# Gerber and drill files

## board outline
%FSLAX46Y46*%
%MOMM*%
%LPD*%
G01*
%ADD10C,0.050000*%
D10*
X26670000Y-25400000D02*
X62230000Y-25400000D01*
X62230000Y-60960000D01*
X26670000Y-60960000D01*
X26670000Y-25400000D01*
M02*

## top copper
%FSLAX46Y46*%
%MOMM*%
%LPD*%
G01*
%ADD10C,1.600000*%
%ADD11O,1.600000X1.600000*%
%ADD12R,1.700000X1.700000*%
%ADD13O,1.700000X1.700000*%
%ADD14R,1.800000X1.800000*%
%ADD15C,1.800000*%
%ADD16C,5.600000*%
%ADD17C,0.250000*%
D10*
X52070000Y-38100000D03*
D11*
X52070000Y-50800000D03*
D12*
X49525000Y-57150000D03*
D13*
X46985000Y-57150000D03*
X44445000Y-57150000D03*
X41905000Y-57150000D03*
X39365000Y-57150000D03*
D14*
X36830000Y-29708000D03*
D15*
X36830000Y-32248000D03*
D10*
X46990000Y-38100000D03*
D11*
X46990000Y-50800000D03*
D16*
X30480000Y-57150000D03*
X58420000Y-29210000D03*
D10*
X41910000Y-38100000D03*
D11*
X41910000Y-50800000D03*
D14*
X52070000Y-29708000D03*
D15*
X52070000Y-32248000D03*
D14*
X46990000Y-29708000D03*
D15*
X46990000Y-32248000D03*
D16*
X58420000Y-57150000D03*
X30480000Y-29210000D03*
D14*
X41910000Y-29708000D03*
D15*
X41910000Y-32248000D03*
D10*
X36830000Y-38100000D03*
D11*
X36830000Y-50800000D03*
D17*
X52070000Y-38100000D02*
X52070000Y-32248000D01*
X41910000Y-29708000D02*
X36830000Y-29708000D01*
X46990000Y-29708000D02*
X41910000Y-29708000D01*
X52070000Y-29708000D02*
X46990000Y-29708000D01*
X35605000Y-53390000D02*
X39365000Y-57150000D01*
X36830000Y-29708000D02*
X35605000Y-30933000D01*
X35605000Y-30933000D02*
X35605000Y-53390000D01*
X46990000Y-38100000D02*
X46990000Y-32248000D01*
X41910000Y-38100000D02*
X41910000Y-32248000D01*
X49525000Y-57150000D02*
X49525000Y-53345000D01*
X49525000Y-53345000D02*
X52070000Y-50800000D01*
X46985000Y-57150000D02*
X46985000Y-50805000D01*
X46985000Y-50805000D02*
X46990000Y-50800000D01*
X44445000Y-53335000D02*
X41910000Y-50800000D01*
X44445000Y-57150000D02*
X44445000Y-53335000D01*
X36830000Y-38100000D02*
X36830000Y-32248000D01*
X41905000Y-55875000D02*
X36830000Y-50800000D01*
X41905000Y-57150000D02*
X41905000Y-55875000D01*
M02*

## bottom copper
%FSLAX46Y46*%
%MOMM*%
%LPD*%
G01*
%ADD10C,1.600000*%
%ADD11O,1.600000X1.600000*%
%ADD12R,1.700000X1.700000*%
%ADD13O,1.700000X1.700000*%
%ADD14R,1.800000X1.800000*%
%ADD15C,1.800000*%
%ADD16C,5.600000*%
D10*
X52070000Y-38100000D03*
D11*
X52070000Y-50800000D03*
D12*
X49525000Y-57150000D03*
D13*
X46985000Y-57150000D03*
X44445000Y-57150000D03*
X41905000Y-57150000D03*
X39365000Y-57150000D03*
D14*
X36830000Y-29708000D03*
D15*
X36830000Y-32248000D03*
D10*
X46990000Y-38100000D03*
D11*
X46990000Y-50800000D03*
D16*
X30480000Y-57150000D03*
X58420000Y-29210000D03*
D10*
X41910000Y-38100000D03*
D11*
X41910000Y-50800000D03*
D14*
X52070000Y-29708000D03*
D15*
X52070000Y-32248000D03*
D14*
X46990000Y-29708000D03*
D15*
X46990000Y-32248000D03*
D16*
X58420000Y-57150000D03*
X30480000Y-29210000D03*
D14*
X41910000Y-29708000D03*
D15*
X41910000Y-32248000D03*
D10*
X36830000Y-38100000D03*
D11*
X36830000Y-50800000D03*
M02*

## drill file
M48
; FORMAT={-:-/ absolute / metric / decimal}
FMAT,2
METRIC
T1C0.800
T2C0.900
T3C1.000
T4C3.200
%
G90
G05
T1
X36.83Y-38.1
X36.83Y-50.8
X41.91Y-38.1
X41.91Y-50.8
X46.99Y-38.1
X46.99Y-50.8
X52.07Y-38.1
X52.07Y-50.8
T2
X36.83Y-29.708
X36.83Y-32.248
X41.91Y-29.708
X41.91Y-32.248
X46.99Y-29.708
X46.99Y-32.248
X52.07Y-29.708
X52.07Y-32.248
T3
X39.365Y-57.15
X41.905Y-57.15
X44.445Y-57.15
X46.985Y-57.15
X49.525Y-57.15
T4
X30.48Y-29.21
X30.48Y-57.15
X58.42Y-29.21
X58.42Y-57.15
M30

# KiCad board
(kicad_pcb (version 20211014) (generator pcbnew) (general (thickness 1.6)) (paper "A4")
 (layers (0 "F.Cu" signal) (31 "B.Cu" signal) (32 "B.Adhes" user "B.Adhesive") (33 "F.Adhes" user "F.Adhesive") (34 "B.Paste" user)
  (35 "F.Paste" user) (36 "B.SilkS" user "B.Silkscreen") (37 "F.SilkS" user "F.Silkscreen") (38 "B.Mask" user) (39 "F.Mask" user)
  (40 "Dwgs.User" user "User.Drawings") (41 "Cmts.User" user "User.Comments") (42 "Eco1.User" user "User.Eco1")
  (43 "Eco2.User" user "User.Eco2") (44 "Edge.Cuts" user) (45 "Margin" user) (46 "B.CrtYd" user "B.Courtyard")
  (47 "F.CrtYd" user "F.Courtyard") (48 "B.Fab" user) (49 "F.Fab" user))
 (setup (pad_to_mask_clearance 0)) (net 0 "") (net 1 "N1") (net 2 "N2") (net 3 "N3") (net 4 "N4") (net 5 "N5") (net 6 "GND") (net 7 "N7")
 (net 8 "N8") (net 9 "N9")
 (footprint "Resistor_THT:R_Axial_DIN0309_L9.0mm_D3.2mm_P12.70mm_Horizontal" (layer "F.Cu") (at 52.07 38.1 -90)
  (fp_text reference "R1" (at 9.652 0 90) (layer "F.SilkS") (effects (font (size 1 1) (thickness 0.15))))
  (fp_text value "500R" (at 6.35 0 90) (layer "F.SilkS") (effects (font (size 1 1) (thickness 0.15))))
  (pad "1" thru_hole circle (at 0 0 270) (size 1.6 1.6) (drill 0.8) (layers *.Cu *.Mask) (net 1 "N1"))
  (pad "2" thru_hole oval (at 12.7 0 270) (size 1.6 1.6) (drill 0.8) (layers *.Cu *.Mask) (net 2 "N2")))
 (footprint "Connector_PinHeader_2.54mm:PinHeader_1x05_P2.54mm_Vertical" (layer "F.Cu") (at 49.525 57.15 -90)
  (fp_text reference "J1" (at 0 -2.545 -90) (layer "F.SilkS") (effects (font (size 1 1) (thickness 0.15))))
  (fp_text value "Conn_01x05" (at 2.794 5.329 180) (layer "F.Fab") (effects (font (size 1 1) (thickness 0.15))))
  (pad "1" thru_hole rect (at 0 0 270) (size 1.7 1.7) (drill 1) (layers *.Cu *.Mask) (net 2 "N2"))
  (pad "2" thru_hole oval (at 0 2.54 270) (size 1.7 1.7) (drill 1) (layers *.Cu *.Mask) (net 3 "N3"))
  (pad "3" thru_hole oval (at 0 5.08 270) (size 1.7 1.7) (drill 1) (layers *.Cu *.Mask) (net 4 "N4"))
  (pad "4" thru_hole oval (at 0 7.62 270) (size 1.7 1.7) (drill 1) (layers *.Cu *.Mask) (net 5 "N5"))
  (pad "5" thru_hole oval (at 0 10.16 270) (size 1.7 1.7) (drill 1) (layers *.Cu *.Mask) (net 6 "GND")))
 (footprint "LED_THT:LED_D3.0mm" (layer "F.Cu") (at 36.83 29.708 -90)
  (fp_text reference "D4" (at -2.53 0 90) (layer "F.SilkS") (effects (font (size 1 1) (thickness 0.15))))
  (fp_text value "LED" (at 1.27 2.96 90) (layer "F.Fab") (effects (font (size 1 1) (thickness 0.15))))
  (pad "1" thru_hole rect (at 0 0 270) (size 1.8 1.8) (drill 0.9) (layers *.Cu *.Mask) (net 6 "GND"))
  (pad "2" thru_hole circle (at 2.54 0 270) (size 1.8 1.8) (drill 0.9) (layers *.Cu *.Mask) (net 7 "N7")))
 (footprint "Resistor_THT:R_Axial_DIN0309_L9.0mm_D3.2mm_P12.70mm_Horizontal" (layer "F.Cu") (at 46.99 38.1 -90)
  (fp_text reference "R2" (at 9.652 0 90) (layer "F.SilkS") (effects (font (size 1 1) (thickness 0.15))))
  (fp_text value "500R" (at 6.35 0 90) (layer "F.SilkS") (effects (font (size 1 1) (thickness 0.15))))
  (pad "1" thru_hole circle (at 0 0 270) (size 1.6 1.6) (drill 0.8) (layers *.Cu *.Mask) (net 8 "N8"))
  (pad "2" thru_hole oval (at 12.7 0 270) (size 1.6 1.6) (drill 0.8) (layers *.Cu *.Mask) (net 3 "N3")))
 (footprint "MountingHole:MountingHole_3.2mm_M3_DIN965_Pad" (layer "F.Cu") (at 30.48 57.15)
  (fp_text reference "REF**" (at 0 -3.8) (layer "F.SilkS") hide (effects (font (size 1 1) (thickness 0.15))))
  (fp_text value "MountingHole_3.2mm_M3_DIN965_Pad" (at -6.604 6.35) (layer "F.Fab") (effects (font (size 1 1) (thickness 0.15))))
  (pad "1" thru_hole circle (at 0 0) (size 5.6 5.6) (drill 3.2) (layers F&B.Cu *.Mask)))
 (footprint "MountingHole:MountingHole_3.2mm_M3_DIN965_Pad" (layer "F.Cu") (at 58.42 29.21)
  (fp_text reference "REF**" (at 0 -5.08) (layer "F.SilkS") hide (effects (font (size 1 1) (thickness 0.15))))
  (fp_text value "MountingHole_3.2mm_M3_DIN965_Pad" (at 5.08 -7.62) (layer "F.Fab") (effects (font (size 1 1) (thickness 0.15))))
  (pad "1" thru_hole circle (at 0 0) (size 5.6 5.6) (drill 3.2) (layers F&B.Cu *.Mask)))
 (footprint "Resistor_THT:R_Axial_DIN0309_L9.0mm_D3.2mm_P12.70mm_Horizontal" (layer "F.Cu") (at 41.91 38.1 -90)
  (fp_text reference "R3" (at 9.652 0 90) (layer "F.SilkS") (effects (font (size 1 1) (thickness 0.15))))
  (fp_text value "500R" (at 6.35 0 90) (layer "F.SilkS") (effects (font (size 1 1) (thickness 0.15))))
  (pad "1" thru_hole circle (at 0 0 270) (size 1.6 1.6) (drill 0.8) (layers *.Cu *.Mask) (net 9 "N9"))
  (pad "2" thru_hole oval (at 12.7 0 270) (size 1.6 1.6) (drill 0.8) (layers *.Cu *.Mask) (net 4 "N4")))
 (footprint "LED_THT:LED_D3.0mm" (layer "F.Cu") (at 52.07 29.708 -90)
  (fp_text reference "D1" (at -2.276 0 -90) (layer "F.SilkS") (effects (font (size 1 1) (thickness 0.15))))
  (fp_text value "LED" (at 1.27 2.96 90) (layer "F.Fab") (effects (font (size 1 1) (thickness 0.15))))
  (pad "1" thru_hole rect (at 0 0 270) (size 1.8 1.8) (drill 0.9) (layers *.Cu *.Mask) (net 6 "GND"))
  (pad "2" thru_hole circle (at 2.54 0 270) (size 1.8 1.8) (drill 0.9) (layers *.Cu *.Mask) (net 1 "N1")))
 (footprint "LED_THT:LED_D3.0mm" (layer "F.Cu") (at 46.99 29.708 -90)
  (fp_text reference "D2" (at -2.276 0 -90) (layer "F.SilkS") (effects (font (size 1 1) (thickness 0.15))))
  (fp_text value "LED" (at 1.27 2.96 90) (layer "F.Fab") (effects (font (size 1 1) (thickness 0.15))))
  (pad "1" thru_hole rect (at 0 0 270) (size 1.8 1.8) (drill 0.9) (layers *.Cu *.Mask) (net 6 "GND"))
  (pad "2" thru_hole circle (at 2.54 0 270) (size 1.8 1.8) (drill 0.9) (layers *.Cu *.Mask) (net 8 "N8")))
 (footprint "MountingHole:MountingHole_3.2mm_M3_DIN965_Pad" (layer "F.Cu") (at 58.42 57.15)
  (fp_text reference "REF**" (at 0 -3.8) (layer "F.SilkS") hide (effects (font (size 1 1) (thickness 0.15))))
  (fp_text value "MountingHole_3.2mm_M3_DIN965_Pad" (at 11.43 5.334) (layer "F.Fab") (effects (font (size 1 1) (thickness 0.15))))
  (pad "1" thru_hole circle (at 0 0) (size 5.6 5.6) (drill 3.2) (layers *.Cu *.Mask)))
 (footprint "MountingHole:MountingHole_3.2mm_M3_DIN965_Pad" (layer "F.Cu") (at 30.48 29.21)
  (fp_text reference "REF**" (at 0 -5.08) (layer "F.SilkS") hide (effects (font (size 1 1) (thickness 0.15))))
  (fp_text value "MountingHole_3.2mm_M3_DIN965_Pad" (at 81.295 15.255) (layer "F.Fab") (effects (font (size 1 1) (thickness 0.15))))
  (pad "1" thru_hole circle (at 0 0) (size 5.6 5.6) (drill 3.2) (layers F&B.Cu *.Mask)))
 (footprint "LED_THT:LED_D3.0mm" (layer "F.Cu") (at 41.91 29.708 -90)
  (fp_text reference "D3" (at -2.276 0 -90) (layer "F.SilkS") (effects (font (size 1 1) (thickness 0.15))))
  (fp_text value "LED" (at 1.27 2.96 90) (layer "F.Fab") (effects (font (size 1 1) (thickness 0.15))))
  (pad "1" thru_hole rect (at 0 0 270) (size 1.8 1.8) (drill 0.9) (layers *.Cu *.Mask) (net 6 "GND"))
  (pad "2" thru_hole circle (at 2.54 0 270) (size 1.8 1.8) (drill 0.9) (layers *.Cu *.Mask) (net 9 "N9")))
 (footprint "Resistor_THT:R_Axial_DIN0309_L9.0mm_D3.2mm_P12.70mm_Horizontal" (layer "F.Cu") (at 36.83 38.1 -90)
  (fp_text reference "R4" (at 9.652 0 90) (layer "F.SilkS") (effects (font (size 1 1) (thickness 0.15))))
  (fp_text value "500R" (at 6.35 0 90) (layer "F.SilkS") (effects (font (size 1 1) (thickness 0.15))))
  (pad "1" thru_hole circle (at 0 0 270) (size 1.6 1.6) (drill 0.8) (layers *.Cu *.Mask) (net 7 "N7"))
  (pad "2" thru_hole oval (at 12.7 0 270) (size 1.6 1.6) (drill 0.8) (layers *.Cu *.Mask) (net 5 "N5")))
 (gr_rect (start 62.23 60.96) (end 26.67 25.4) (layer "Edge.Cuts") (width 0.05) (fill none))
 (segment (start 52.07 38.1) (end 52.07 32.248) (width 0.25) (layer "F.Cu") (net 1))
 (segment (start 41.91 29.708) (end 36.83 29.708) (width 0.25) (layer "F.Cu") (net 6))
 (segment (start 46.99 29.708) (end 41.91 29.708) (width 0.25) (layer "F.Cu") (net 6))
 (segment (start 52.07 29.708) (end 46.99 29.708) (width 0.25) (layer "F.Cu") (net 6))
 (segment (start 35.605 53.39) (end 39.365 57.15) (width 0.25) (layer "F.Cu") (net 6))
 (segment (start 36.83 29.708) (end 35.605 30.933) (width 0.25) (layer "F.Cu") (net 6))
 (segment (start 35.605 30.933) (end 35.605 53.39) (width 0.25) (layer "F.Cu") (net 6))
 (segment (start 46.99 38.1) (end 46.99 32.248) (width 0.25) (layer "F.Cu") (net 8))
 (segment (start 41.91 38.1) (end 41.91 32.248) (width 0.25) (layer "F.Cu") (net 9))
 (segment (start 49.525 57.15) (end 49.525 53.345) (width 0.25) (layer "F.Cu") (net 2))
 (segment (start 49.525 53.345) (end 52.07 50.8) (width 0.25) (layer "F.Cu") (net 2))
 (segment (start 46.985 57.15) (end 46.985 50.805) (width 0.25) (layer "F.Cu") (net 3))
 (segment (start 46.985 50.805) (end 46.99 50.8) (width 0.25) (layer "F.Cu") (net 3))
 (segment (start 44.445 53.335) (end 41.91 50.8) (width 0.25) (layer "F.Cu") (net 4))
 (segment (start 44.445 57.15) (end 44.445 53.335) (width 0.25) (layer "F.Cu") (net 4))
 (segment (start 36.83 38.1) (end 36.83 32.248) (width 0.25) (layer "F.Cu") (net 7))
 (segment (start 41.905 55.875) (end 36.83 50.8) (width 0.25) (layer "F.Cu") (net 5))
 (segment (start 41.905 57.15) (end 41.905 55.875) (width 0.25) (layer "F.Cu") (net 5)))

